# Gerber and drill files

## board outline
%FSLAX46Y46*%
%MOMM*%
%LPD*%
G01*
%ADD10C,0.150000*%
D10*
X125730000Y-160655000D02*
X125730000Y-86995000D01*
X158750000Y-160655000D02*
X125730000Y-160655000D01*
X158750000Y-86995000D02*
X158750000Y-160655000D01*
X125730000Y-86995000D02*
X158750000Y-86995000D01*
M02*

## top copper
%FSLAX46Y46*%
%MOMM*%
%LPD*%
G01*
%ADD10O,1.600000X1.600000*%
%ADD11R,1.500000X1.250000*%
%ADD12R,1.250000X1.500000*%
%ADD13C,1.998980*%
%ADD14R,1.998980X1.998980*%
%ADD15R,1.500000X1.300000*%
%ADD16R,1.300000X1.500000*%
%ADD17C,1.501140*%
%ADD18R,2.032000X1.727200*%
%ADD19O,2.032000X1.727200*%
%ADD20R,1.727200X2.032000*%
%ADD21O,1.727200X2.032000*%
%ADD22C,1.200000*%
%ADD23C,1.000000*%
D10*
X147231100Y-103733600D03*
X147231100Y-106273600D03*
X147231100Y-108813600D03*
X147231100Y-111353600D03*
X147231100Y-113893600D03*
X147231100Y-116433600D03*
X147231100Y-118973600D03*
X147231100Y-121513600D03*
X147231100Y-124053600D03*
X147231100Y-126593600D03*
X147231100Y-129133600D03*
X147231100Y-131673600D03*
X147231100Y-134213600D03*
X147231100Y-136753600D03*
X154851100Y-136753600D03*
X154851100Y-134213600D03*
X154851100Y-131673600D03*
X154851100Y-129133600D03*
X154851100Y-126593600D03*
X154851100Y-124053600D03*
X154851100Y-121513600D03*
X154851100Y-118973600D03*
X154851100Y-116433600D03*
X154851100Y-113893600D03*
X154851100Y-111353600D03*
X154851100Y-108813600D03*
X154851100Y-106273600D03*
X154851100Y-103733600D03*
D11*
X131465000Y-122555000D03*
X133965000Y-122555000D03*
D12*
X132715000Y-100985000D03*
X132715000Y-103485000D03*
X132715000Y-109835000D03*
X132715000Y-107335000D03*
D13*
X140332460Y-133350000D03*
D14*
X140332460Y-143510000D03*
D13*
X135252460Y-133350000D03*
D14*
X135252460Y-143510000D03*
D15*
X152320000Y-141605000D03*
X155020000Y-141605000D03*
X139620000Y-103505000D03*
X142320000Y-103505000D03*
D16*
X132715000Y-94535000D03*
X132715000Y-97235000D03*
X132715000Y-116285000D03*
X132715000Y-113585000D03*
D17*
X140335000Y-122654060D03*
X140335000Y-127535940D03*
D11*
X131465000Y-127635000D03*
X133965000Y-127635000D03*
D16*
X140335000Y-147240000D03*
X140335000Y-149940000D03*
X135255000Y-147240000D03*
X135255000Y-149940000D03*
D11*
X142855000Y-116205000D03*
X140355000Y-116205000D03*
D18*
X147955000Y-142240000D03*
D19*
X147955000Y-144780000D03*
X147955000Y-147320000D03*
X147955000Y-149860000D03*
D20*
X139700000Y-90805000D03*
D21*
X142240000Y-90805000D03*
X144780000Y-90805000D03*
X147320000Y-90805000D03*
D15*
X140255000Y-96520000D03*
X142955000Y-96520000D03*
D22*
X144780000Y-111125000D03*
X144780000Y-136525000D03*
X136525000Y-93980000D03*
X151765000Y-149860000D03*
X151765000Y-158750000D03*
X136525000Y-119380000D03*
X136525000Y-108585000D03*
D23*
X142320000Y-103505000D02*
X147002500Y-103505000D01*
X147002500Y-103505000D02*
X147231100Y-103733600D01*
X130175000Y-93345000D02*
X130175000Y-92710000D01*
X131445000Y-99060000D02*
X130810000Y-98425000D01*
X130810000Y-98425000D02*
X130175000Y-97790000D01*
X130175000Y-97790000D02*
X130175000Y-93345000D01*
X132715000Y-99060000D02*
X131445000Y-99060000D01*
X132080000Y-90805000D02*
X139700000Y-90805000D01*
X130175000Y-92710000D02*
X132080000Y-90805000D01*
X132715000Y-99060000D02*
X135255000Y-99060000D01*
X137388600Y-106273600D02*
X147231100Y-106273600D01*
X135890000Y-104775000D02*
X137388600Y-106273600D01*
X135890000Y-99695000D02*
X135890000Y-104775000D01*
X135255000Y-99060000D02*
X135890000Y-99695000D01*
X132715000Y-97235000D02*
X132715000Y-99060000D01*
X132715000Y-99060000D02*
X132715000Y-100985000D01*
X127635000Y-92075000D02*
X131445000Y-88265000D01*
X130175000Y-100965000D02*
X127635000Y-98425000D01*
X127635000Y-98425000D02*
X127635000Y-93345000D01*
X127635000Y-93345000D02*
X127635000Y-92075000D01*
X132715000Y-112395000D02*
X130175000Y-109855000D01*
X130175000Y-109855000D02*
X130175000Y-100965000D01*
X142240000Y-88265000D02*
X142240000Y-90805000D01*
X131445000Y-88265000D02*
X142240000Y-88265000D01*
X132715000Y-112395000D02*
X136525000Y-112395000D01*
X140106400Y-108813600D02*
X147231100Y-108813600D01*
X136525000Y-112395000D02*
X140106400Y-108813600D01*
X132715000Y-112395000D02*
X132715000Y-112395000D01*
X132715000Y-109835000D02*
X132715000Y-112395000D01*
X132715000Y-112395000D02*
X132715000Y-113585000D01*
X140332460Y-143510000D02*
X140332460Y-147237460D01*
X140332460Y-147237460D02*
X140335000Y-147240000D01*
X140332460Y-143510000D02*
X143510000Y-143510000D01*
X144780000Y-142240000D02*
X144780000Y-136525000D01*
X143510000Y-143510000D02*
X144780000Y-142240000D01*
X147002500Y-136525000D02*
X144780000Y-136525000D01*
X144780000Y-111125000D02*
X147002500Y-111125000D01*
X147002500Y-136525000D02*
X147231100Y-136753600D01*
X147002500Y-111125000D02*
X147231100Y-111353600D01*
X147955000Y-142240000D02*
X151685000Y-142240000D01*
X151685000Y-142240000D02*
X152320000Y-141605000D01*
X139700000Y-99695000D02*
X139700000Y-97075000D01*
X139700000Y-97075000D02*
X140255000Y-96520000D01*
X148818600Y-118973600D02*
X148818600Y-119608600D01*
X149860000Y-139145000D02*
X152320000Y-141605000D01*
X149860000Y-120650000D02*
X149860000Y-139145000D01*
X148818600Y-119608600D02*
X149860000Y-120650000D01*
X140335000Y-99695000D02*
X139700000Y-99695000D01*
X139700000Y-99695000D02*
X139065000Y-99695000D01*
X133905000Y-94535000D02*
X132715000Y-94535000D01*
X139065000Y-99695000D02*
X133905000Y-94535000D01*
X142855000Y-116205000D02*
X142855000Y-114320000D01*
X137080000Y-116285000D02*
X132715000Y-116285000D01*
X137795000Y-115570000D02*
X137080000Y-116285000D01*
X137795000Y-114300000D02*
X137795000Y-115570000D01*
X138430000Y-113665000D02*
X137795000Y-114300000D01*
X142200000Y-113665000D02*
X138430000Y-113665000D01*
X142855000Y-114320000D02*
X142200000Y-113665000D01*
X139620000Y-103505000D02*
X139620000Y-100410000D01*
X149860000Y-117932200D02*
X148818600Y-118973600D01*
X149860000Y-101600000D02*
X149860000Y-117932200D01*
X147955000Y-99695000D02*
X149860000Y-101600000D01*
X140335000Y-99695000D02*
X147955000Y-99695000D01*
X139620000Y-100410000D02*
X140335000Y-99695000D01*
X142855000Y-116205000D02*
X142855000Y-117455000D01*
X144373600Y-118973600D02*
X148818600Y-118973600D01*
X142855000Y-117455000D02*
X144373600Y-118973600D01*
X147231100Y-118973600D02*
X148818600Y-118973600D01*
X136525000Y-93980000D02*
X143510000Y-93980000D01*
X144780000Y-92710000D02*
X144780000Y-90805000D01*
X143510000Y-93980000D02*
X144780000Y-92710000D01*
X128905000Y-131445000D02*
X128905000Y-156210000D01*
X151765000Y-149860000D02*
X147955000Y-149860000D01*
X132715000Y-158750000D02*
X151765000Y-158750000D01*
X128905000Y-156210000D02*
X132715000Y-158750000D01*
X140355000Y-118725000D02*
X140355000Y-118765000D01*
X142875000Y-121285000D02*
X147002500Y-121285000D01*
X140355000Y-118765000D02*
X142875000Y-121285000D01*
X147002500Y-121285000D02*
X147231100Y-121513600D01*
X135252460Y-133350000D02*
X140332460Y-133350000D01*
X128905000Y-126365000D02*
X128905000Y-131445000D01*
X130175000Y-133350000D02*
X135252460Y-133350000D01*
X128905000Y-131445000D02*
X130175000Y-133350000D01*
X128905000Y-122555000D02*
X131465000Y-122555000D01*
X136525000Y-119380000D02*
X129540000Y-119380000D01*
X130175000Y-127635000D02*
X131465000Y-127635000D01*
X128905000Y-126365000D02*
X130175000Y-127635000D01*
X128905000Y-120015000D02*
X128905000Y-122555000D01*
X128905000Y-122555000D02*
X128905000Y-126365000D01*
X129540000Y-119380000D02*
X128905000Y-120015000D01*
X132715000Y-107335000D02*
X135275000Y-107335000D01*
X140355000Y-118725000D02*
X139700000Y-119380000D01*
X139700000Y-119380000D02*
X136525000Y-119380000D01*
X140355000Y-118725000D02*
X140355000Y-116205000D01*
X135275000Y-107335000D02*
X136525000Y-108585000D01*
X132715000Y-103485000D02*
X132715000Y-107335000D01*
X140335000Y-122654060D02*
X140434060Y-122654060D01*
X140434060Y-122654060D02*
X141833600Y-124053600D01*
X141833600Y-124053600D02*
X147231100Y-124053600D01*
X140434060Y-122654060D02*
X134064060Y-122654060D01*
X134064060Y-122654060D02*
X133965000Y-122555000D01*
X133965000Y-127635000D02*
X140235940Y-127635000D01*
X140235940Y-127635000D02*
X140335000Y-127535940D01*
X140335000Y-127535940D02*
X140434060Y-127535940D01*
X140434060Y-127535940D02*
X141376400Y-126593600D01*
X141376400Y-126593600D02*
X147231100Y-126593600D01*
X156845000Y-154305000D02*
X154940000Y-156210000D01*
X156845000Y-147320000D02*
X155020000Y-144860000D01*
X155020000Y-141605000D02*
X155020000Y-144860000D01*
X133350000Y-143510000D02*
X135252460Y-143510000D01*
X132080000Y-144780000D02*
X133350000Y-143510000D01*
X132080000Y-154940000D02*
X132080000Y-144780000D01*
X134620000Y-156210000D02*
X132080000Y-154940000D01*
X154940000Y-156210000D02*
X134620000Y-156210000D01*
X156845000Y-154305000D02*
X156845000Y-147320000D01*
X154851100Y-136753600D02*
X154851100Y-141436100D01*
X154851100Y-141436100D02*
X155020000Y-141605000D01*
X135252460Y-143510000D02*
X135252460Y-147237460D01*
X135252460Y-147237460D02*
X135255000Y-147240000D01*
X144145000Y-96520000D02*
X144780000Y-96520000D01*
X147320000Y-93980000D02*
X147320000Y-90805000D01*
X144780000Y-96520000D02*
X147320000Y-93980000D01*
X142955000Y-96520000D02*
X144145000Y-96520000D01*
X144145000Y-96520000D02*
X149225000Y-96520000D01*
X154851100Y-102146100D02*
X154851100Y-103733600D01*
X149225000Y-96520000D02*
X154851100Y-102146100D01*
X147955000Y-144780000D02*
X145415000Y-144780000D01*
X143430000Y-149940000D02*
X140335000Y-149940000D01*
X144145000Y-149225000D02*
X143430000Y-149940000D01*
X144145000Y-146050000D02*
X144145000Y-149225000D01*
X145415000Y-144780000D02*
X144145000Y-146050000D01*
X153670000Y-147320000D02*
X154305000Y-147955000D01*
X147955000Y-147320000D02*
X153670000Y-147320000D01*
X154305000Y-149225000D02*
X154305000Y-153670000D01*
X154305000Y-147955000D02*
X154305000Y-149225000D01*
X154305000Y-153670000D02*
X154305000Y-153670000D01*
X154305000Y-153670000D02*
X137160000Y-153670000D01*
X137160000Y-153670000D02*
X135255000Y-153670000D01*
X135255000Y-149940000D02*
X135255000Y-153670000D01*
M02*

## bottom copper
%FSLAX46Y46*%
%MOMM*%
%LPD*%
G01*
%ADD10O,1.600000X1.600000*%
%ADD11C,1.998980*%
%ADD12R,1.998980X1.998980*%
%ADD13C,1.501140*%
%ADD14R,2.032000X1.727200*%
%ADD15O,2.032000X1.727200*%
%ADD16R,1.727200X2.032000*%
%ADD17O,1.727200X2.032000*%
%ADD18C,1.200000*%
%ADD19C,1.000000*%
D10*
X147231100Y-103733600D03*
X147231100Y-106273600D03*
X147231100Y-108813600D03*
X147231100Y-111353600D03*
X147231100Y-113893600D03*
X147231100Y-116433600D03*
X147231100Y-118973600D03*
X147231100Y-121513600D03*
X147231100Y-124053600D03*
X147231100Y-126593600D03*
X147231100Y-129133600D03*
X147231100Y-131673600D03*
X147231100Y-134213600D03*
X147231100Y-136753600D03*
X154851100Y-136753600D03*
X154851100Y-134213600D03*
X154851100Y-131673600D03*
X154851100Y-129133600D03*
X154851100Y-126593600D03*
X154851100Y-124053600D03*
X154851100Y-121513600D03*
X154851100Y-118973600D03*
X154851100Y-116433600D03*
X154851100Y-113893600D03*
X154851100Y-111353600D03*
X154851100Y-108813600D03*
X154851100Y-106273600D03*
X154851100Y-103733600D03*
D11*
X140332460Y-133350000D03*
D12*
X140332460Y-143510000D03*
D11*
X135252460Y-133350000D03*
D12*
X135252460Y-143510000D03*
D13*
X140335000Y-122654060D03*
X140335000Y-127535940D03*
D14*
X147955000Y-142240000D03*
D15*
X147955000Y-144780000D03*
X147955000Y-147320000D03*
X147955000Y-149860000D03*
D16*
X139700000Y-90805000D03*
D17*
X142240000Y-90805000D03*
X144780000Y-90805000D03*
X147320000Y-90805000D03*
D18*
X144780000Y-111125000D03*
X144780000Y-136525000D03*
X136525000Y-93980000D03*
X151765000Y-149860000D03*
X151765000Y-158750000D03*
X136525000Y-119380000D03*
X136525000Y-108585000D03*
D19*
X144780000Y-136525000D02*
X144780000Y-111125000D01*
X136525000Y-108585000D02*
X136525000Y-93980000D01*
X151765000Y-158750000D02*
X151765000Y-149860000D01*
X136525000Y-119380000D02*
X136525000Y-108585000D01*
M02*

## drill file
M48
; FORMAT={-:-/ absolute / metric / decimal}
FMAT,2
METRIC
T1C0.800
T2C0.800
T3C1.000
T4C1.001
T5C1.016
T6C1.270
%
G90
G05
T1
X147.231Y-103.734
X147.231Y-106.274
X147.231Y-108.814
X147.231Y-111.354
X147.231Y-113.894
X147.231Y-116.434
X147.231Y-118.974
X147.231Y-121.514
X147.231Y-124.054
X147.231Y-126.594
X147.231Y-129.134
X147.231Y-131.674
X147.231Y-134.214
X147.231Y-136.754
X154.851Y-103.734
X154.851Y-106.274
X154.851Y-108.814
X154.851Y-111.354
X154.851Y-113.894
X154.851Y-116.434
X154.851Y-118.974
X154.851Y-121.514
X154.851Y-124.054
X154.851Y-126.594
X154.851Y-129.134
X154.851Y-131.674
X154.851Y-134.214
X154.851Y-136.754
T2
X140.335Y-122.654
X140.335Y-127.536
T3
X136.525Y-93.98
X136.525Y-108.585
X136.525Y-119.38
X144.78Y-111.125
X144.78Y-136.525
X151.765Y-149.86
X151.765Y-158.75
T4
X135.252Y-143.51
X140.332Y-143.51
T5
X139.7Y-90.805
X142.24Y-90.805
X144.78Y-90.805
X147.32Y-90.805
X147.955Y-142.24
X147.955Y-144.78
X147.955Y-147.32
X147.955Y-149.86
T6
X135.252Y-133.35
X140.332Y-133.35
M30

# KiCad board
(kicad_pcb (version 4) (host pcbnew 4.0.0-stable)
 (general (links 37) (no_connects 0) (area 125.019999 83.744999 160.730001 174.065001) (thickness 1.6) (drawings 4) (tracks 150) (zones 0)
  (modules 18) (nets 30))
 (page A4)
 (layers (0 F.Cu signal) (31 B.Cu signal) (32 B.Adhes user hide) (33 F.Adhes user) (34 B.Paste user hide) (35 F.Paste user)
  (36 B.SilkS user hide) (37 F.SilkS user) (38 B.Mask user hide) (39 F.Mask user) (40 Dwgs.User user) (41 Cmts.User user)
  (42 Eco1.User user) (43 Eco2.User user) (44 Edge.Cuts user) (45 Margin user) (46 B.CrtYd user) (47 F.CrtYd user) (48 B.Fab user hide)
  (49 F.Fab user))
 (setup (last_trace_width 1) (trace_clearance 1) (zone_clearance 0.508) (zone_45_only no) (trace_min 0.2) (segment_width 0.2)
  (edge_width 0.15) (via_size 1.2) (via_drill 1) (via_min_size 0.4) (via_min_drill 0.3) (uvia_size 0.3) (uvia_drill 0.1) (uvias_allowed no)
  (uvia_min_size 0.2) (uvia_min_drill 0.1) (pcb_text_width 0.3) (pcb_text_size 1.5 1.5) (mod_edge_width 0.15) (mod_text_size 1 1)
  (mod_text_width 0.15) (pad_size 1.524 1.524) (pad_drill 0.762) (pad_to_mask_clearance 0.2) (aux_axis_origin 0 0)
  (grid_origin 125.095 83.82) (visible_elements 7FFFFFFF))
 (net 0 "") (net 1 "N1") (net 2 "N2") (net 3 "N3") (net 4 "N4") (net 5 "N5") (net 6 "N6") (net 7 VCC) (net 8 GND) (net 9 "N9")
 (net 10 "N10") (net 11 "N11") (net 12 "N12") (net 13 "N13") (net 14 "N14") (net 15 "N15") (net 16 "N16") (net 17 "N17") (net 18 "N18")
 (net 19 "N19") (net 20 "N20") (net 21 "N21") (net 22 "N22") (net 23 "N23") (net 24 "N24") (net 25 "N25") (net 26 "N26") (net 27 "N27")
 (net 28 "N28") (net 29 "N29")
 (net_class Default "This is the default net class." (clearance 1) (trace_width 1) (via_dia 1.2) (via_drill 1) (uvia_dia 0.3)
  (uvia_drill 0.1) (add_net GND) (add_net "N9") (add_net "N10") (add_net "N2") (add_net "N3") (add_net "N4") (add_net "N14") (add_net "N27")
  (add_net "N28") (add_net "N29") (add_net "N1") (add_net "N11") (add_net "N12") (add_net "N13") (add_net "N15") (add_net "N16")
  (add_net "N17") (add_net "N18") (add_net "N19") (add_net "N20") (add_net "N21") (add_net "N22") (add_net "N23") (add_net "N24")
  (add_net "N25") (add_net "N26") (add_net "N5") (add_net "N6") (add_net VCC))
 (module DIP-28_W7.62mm (layer F.Cu) (at 147.2311 103.7336)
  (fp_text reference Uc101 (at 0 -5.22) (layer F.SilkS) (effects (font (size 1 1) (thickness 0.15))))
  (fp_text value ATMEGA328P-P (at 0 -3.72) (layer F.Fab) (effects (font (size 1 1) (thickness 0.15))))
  (pad 1 thru_hole oval (at 0 0) (size 1.6 1.6) (drill 0.8) (layers *.Cu *.Mask F.SilkS) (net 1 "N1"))
  (pad 2 thru_hole oval (at 0 2.54) (size 1.6 1.6) (drill 0.8) (layers *.Cu *.Mask F.SilkS) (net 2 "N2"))
  (pad 3 thru_hole oval (at 0 5.08) (size 1.6 1.6) (drill 0.8) (layers *.Cu *.Mask F.SilkS) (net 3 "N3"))
  (pad 4 thru_hole oval (at 0 7.62) (size 1.6 1.6) (drill 0.8) (layers *.Cu *.Mask F.SilkS) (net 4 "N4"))
  (pad 5 thru_hole oval (at 0 10.16) (size 1.6 1.6) (drill 0.8) (layers *.Cu *.Mask F.SilkS) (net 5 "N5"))
  (pad 6 thru_hole oval (at 0 12.7) (size 1.6 1.6) (drill 0.8) (layers *.Cu *.Mask F.SilkS) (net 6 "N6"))
  (pad 7 thru_hole oval (at 0 15.24) (size 1.6 1.6) (drill 0.8) (layers *.Cu *.Mask F.SilkS) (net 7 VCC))
  (pad 8 thru_hole oval (at 0 17.78) (size 1.6 1.6) (drill 0.8) (layers *.Cu *.Mask F.SilkS) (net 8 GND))
  (pad 9 thru_hole oval (at 0 20.32) (size 1.6 1.6) (drill 0.8) (layers *.Cu *.Mask F.SilkS) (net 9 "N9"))
  (pad 10 thru_hole oval (at 0 22.86) (size 1.6 1.6) (drill 0.8) (layers *.Cu *.Mask F.SilkS) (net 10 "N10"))
  (pad 11 thru_hole oval (at 0 25.4) (size 1.6 1.6) (drill 0.8) (layers *.Cu *.Mask F.SilkS) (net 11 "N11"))
  (pad 12 thru_hole oval (at 0 27.94) (size 1.6 1.6) (drill 0.8) (layers *.Cu *.Mask F.SilkS) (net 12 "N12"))
  (pad 13 thru_hole oval (at 0 30.48) (size 1.6 1.6) (drill 0.8) (layers *.Cu *.Mask F.SilkS) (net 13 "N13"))
  (pad 14 thru_hole oval (at 0 33.02) (size 1.6 1.6) (drill 0.8) (layers *.Cu *.Mask F.SilkS) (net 4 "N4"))
  (pad 15 thru_hole oval (at 7.62 33.02) (size 1.6 1.6) (drill 0.8) (layers *.Cu *.Mask F.SilkS) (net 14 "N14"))
  (pad 16 thru_hole oval (at 7.62 30.48) (size 1.6 1.6) (drill 0.8) (layers *.Cu *.Mask F.SilkS) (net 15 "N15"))
  (pad 17 thru_hole oval (at 7.62 27.94) (size 1.6 1.6) (drill 0.8) (layers *.Cu *.Mask F.SilkS) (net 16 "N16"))
  (pad 18 thru_hole oval (at 7.62 25.4) (size 1.6 1.6) (drill 0.8) (layers *.Cu *.Mask F.SilkS) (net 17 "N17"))
  (pad 19 thru_hole oval (at 7.62 22.86) (size 1.6 1.6) (drill 0.8) (layers *.Cu *.Mask F.SilkS) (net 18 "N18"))
  (pad 20 thru_hole oval (at 7.62 20.32) (size 1.6 1.6) (drill 0.8) (layers *.Cu *.Mask F.SilkS) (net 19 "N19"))
  (pad 21 thru_hole oval (at 7.62 17.78) (size 1.6 1.6) (drill 0.8) (layers *.Cu *.Mask F.SilkS) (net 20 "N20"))
  (pad 22 thru_hole oval (at 7.62 15.24) (size 1.6 1.6) (drill 0.8) (layers *.Cu *.Mask F.SilkS) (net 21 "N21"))
  (pad 23 thru_hole oval (at 7.62 12.7) (size 1.6 1.6) (drill 0.8) (layers *.Cu *.Mask F.SilkS) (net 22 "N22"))
  (pad 24 thru_hole oval (at 7.62 10.16) (size 1.6 1.6) (drill 0.8) (layers *.Cu *.Mask F.SilkS) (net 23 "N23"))
  (pad 25 thru_hole oval (at 7.62 7.62) (size 1.6 1.6) (drill 0.8) (layers *.Cu *.Mask F.SilkS) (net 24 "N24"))
  (pad 26 thru_hole oval (at 7.62 5.08) (size 1.6 1.6) (drill 0.8) (layers *.Cu *.Mask F.SilkS) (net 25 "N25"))
  (pad 27 thru_hole oval (at 7.62 2.54) (size 1.6 1.6) (drill 0.8) (layers *.Cu *.Mask F.SilkS) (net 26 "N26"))
  (pad 28 thru_hole oval (at 7.62 0) (size 1.6 1.6) (drill 0.8) (layers *.Cu *.Mask F.SilkS) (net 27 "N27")))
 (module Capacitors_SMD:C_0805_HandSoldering (layer F.Cu) (at 132.715 122.555)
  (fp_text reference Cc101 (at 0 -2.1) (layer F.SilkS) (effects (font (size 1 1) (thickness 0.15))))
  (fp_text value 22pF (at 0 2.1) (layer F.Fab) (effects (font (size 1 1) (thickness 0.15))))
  (pad 1 smd rect (at -1.25 0) (size 1.5 1.25) (layers F.Cu F.Paste F.Mask) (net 8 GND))
  (pad 2 smd rect (at 1.25 0) (size 1.5 1.25) (layers F.Cu F.Paste F.Mask) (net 9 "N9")))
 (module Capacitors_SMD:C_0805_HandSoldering (layer F.Cu) (at 132.715 102.235 270)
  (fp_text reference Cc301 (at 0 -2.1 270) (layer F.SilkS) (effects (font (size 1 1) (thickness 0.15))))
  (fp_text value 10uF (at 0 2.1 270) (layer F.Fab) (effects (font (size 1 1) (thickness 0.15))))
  (pad 1 smd rect (at -1.25 0 270) (size 1.5 1.25) (layers F.Cu F.Paste F.Mask) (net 2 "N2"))
  (pad 2 smd rect (at 1.25 0 270) (size 1.5 1.25) (layers F.Cu F.Paste F.Mask) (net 8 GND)))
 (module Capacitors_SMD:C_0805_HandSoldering (layer F.Cu) (at 132.715 108.585 90)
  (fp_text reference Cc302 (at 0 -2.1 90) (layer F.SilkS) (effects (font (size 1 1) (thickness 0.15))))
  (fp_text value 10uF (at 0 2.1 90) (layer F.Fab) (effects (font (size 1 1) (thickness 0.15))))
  (pad 1 smd rect (at -1.25 0 90) (size 1.5 1.25) (layers F.Cu F.Paste F.Mask) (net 3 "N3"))
  (pad 2 smd rect (at 1.25 0 90) (size 1.5 1.25) (layers F.Cu F.Paste F.Mask) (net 8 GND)))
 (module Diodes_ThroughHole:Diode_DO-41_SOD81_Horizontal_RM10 (layer F.Cu) (at 140.335 143.51 90)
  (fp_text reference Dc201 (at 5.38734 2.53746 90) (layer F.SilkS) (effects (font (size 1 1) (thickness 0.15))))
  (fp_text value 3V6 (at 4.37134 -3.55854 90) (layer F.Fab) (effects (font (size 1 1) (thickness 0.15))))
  (pad 2 thru_hole circle (at 10.16 -0.00254 270) (size 1.99898 1.99898) (drill 1.27) (layers *.Cu *.Mask F.SilkS) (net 8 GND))
  (pad 1 thru_hole rect (at 0 -0.00254 270) (size 1.99898 1.99898) (drill 1.00076) (layers *.Cu *.Mask F.SilkS) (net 4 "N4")))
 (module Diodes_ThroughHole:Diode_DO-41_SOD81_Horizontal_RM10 (layer F.Cu) (at 135.255 143.51 90)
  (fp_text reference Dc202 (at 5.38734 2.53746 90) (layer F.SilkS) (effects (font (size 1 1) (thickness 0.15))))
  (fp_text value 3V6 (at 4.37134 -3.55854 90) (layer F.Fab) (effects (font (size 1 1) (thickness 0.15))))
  (pad 2 thru_hole circle (at 10.16 -0.00254 270) (size 1.99898 1.99898) (drill 1.27) (layers *.Cu *.Mask F.SilkS) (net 8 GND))
  (pad 1 thru_hole rect (at 0 -0.00254 270) (size 1.99898 1.99898) (drill 1.00076) (layers *.Cu *.Mask F.SilkS) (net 14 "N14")))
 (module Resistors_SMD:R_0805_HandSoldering (layer F.Cu) (at 153.67 141.605)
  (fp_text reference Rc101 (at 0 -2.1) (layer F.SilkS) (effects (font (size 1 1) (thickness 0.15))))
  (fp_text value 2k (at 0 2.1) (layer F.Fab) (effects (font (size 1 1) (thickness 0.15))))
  (pad 1 smd rect (at -1.35 0) (size 1.5 1.3) (layers F.Cu F.Paste F.Mask) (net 7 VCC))
  (pad 2 smd rect (at 1.35 0) (size 1.5 1.3) (layers F.Cu F.Paste F.Mask) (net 14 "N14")))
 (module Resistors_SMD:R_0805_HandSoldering (layer F.Cu) (at 140.97 103.505)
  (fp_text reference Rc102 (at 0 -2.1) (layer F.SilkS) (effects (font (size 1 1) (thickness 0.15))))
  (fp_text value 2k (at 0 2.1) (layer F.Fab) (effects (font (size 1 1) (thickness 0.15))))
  (pad 1 smd rect (at -1.35 0) (size 1.5 1.3) (layers F.Cu F.Paste F.Mask) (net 7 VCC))
  (pad 2 smd rect (at 1.35 0) (size 1.5 1.3) (layers F.Cu F.Paste F.Mask) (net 1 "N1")))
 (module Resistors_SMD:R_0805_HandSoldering (layer F.Cu) (at 132.715 95.885 270)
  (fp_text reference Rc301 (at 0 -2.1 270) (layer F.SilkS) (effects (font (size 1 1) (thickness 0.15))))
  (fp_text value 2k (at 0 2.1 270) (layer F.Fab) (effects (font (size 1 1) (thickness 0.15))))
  (pad 1 smd rect (at -1.35 0 270) (size 1.5 1.3) (layers F.Cu F.Paste F.Mask) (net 7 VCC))
  (pad 2 smd rect (at 1.35 0 270) (size 1.5 1.3) (layers F.Cu F.Paste F.Mask) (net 2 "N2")))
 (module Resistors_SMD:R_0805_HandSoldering (layer F.Cu) (at 132.715 114.935 90)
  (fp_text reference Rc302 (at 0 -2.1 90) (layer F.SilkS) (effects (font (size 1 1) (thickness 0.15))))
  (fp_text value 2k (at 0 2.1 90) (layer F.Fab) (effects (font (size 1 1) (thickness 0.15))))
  (pad 1 smd rect (at -1.35 0 90) (size 1.5 1.3) (layers F.Cu F.Paste F.Mask) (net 7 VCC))
  (pad 2 smd rect (at 1.35 0 90) (size 1.5 1.3) (layers F.Cu F.Paste F.Mask) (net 3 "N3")))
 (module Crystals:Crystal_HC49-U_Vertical (layer F.Cu) (at 140.335 125.095 270)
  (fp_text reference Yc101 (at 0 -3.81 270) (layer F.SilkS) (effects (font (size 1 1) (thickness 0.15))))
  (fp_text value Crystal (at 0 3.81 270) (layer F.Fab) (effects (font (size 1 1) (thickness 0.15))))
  (pad 1 thru_hole circle (at -2.44094 0 270) (size 1.50114 1.50114) (drill 0.8001) (layers *.Cu *.Mask F.SilkS) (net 9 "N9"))
  (pad 2 thru_hole circle (at 2.44094 0 270) (size 1.50114 1.50114) (drill 0.8001) (layers *.Cu *.Mask F.SilkS) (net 10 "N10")))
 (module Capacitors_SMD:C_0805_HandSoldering (layer F.Cu) (at 132.715 127.635)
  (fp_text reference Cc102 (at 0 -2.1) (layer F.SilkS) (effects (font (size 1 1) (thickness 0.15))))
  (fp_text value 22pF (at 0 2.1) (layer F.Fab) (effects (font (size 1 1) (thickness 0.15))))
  (pad 1 smd rect (at -1.25 0) (size 1.5 1.25) (layers F.Cu F.Paste F.Mask) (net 8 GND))
  (pad 2 smd rect (at 1.25 0) (size 1.5 1.25) (layers F.Cu F.Paste F.Mask) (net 10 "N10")))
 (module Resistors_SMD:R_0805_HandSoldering (layer F.Cu) (at 140.335 148.59 270)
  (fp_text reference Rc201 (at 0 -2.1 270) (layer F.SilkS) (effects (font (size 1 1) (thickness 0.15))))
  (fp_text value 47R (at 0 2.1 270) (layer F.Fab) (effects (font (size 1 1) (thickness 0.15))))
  (pad 1 smd rect (at -1.35 0 270) (size 1.5 1.3) (layers F.Cu F.Paste F.Mask) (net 4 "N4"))
  (pad 2 smd rect (at 1.35 0 270) (size 1.5 1.3) (layers F.Cu F.Paste F.Mask) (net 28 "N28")))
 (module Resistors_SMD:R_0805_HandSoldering (layer F.Cu) (at 135.255 148.59 270)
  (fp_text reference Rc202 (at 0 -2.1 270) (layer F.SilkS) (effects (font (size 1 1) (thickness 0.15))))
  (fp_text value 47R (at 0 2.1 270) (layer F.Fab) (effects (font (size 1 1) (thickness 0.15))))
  (pad 1 smd rect (at -1.35 0 270) (size 1.5 1.3) (layers F.Cu F.Paste F.Mask) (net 14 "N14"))
  (pad 2 smd rect (at 1.35 0 270) (size 1.5 1.3) (layers F.Cu F.Paste F.Mask) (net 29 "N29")))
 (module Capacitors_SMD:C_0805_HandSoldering (layer F.Cu) (at 141.605 116.205 180)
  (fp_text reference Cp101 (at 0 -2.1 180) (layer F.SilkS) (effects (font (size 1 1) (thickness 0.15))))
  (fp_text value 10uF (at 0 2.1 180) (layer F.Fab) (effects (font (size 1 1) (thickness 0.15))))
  (pad 1 smd rect (at -1.25 0 180) (size 1.5 1.25) (layers F.Cu F.Paste F.Mask) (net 7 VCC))
  (pad 2 smd rect (at 1.25 0 180) (size 1.5 1.25) (layers F.Cu F.Paste F.Mask) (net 8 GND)))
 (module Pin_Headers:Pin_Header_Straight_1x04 (layer F.Cu) (at 147.955 142.24)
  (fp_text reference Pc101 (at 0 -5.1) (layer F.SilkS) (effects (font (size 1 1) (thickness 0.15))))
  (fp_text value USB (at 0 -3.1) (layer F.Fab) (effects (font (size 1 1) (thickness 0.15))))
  (pad 1 thru_hole rect (at 0 0) (size 2.032 1.7272) (drill 1.016) (layers *.Cu *.Mask F.SilkS) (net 7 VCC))
  (pad 2 thru_hole oval (at 0 2.54) (size 2.032 1.7272) (drill 1.016) (layers *.Cu *.Mask F.SilkS) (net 28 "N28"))
  (pad 3 thru_hole oval (at 0 5.08) (size 2.032 1.7272) (drill 1.016) (layers *.Cu *.Mask F.SilkS) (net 29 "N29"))
  (pad 4 thru_hole oval (at 0 7.62) (size 2.032 1.7272) (drill 1.016) (layers *.Cu *.Mask F.SilkS) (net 8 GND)))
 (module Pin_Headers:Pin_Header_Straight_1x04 (layer F.Cu) (at 139.7 90.805 90)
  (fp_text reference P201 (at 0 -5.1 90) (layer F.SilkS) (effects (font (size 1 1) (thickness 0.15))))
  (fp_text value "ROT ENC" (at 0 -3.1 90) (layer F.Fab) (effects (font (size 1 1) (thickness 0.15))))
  (pad 1 thru_hole rect (at 0 0 90) (size 2.032 1.7272) (drill 1.016) (layers *.Cu *.Mask F.SilkS) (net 2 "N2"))
  (pad 2 thru_hole oval (at 0 2.54 90) (size 2.032 1.7272) (drill 1.016) (layers *.Cu *.Mask F.SilkS) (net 3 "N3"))
  (pad 3 thru_hole oval (at 0 5.08 90) (size 2.032 1.7272) (drill 1.016) (layers *.Cu *.Mask F.SilkS) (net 8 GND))
  (pad 4 thru_hole oval (at 0 7.62 90) (size 2.032 1.7272) (drill 1.016) (layers *.Cu *.Mask F.SilkS) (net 27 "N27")))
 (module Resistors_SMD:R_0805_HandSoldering (layer F.Cu) (at 141.605 96.52)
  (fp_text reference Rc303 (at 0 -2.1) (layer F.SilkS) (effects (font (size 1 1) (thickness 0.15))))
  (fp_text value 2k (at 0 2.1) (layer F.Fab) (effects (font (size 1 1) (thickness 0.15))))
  (pad 1 smd rect (at -1.35 0) (size 1.5 1.3) (layers F.Cu F.Paste F.Mask) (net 7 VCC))
  (pad 2 smd rect (at 1.35 0) (size 1.5 1.3) (layers F.Cu F.Paste F.Mask) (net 27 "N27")))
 (gr_line (start 125.73 160.655) (end 125.73 86.995) (angle 90) (layer Edge.Cuts) (width 0.15))
 (gr_line (start 158.75 160.655) (end 125.73 160.655) (angle 90) (layer Edge.Cuts) (width 0.15))
 (gr_line (start 158.75 86.995) (end 158.75 160.655) (angle 90) (layer Edge.Cuts) (width 0.15))
 (gr_line (start 125.73 86.995) (end 158.75 86.995) (angle 90) (layer Edge.Cuts) (width 0.15))
 (segment (start 142.32 103.505) (end 147.0025 103.505) (width 1) (layer F.Cu) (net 1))
 (segment (start 147.0025 103.505) (end 147.2311 103.7336) (width 1) (layer F.Cu) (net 1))
 (segment (start 130.175 93.345) (end 130.175 92.71) (width 1) (layer F.Cu) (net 2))
 (segment (start 131.445 99.06) (end 130.81 98.425) (width 1) (layer F.Cu) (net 2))
 (segment (start 130.81 98.425) (end 130.175 97.79) (width 1) (layer F.Cu) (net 2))
 (segment (start 130.175 97.79) (end 130.175 93.345) (width 1) (layer F.Cu) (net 2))
 (segment (start 132.715 99.06) (end 131.445 99.06) (width 1) (layer F.Cu) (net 2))
 (segment (start 132.08 90.805) (end 139.7 90.805) (width 1) (layer F.Cu) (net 2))
 (segment (start 130.175 92.71) (end 132.08 90.805) (width 1) (layer F.Cu) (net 2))
 (segment (start 132.715 99.06) (end 135.255 99.06) (width 1) (layer F.Cu) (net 2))
 (segment (start 137.3886 106.2736) (end 147.2311 106.2736) (width 1) (layer F.Cu) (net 2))
 (segment (start 135.89 104.775) (end 137.3886 106.2736) (width 1) (layer F.Cu) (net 2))
 (segment (start 135.89 99.695) (end 135.89 104.775) (width 1) (layer F.Cu) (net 2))
 (segment (start 135.255 99.06) (end 135.89 99.695) (width 1) (layer F.Cu) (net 2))
 (segment (start 132.715 97.235) (end 132.715 99.06) (width 1) (layer F.Cu) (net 2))
 (segment (start 132.715 99.06) (end 132.715 100.985) (width 1) (layer F.Cu) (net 2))
 (segment (start 127.635 92.075) (end 131.445 88.265) (width 1) (layer F.Cu) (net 3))
 (segment (start 130.175 100.965) (end 127.635 98.425) (width 1) (layer F.Cu) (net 3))
 (segment (start 127.635 98.425) (end 127.635 93.345) (width 1) (layer F.Cu) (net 3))
 (segment (start 127.635 93.345) (end 127.635 92.075) (width 1) (layer F.Cu) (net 3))
 (segment (start 132.715 112.395) (end 130.175 109.855) (width 1) (layer F.Cu) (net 3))
 (segment (start 130.175 109.855) (end 130.175 100.965) (width 1) (layer F.Cu) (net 3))
 (segment (start 142.24 88.265) (end 142.24 90.805) (width 1) (layer F.Cu) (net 3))
 (segment (start 131.445 88.265) (end 142.24 88.265) (width 1) (layer F.Cu) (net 3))
 (segment (start 132.715 112.395) (end 136.525 112.395) (width 1) (layer F.Cu) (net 3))
 (segment (start 140.1064 108.8136) (end 147.2311 108.8136) (width 1) (layer F.Cu) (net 3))
 (segment (start 136.525 112.395) (end 140.1064 108.8136) (width 1) (layer F.Cu) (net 3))
 (segment (start 132.715 112.395) (end 132.715 112.395) (width 1) (layer F.Cu) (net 3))
 (segment (start 132.715 109.835) (end 132.715 112.395) (width 1) (layer F.Cu) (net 3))
 (segment (start 132.715 112.395) (end 132.715 113.585) (width 1) (layer F.Cu) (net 3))
 (segment (start 140.33246 143.51) (end 140.33246 147.23746) (width 1) (layer F.Cu) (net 4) (status 20))
 (segment (start 140.33246 147.23746) (end 140.335 147.24) (width 1) (layer F.Cu) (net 4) (status 30))
 (segment (start 140.33246 143.51) (end 143.51 143.51) (width 1) (layer F.Cu) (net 4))
 (segment (start 144.78 142.24) (end 144.78 136.525) (width 1) (layer F.Cu) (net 4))
 (segment (start 143.51 143.51) (end 144.78 142.24) (width 1) (layer F.Cu) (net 4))
 (segment (start 147.0025 136.525) (end 144.78 136.525) (width 1) (layer F.Cu) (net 4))
 (via (at 144.78 111.125) (size 1.2) (drill 1) (layers F.Cu B.Cu) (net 4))
 (segment (start 144.78 136.525) (end 144.78 111.125) (width 1) (layer B.Cu) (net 4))
 (via (at 144.78 136.525) (size 1.2) (drill 1) (layers F.Cu B.Cu) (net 4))
 (segment (start 144.78 111.125) (end 147.0025 111.125) (width 1) (layer F.Cu) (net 4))
 (segment (start 147.0025 136.525) (end 147.2311 136.7536) (width 1) (layer F.Cu) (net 4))
 (segment (start 147.0025 111.125) (end 147.2311 111.3536) (width 1) (layer F.Cu) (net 4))
 (segment (start 147.955 142.24) (end 151.685 142.24) (width 1) (layer F.Cu) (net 7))
 (segment (start 151.685 142.24) (end 152.32 141.605) (width 1) (layer F.Cu) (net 7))
 (segment (start 139.7 99.695) (end 139.7 97.075) (width 1) (layer F.Cu) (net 7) (status 20))
 (segment (start 139.7 97.075) (end 140.255 96.52) (width 1) (layer F.Cu) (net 7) (status 30))
 (segment (start 148.8186 118.9736) (end 148.8186 119.6086) (width 1) (layer F.Cu) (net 7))
 (segment (start 149.86 139.145) (end 152.32 141.605) (width 1) (layer F.Cu) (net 7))
 (segment (start 149.86 120.65) (end 149.86 139.145) (width 1) (layer F.Cu) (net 7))
 (segment (start 148.8186 119.6086) (end 149.86 120.65) (width 1) (layer F.Cu) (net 7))
 (segment (start 140.335 99.695) (end 139.7 99.695) (width 1) (layer F.Cu) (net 7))
 (segment (start 139.7 99.695) (end 139.065 99.695) (width 1) (layer F.Cu) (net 7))
 (segment (start 133.905 94.535) (end 132.715 94.535) (width 1) (layer F.Cu) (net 7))
 (segment (start 139.065 99.695) (end 133.905 94.535) (width 1) (layer F.Cu) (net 7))
 (segment (start 142.855 116.205) (end 142.855 114.32) (width 1) (layer F.Cu) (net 7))
 (segment (start 137.08 116.285) (end 132.715 116.285) (width 1) (layer F.Cu) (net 7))
 (segment (start 137.795 115.57) (end 137.08 116.285) (width 1) (layer F.Cu) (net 7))
 (segment (start 137.795 114.3) (end 137.795 115.57) (width 1) (layer F.Cu) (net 7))
 (segment (start 138.43 113.665) (end 137.795 114.3) (width 1) (layer F.Cu) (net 7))
 (segment (start 142.2 113.665) (end 138.43 113.665) (width 1) (layer F.Cu) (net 7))
 (segment (start 142.855 114.32) (end 142.2 113.665) (width 1) (layer F.Cu) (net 7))
 (segment (start 139.62 103.505) (end 139.62 100.41) (width 1) (layer F.Cu) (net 7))
 (segment (start 149.86 117.9322) (end 148.8186 118.9736) (width 1) (layer F.Cu) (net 7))
 (segment (start 149.86 101.6) (end 149.86 117.9322) (width 1) (layer F.Cu) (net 7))
 (segment (start 147.955 99.695) (end 149.86 101.6) (width 1) (layer F.Cu) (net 7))
 (segment (start 140.335 99.695) (end 147.955 99.695) (width 1) (layer F.Cu) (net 7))
 (segment (start 139.62 100.41) (end 140.335 99.695) (width 1) (layer F.Cu) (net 7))
 (segment (start 142.855 116.205) (end 142.855 117.455) (width 1) (layer F.Cu) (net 7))
 (segment (start 144.3736 118.9736) (end 148.8186 118.9736) (width 1) (layer F.Cu) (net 7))
 (segment (start 142.855 117.455) (end 144.3736 118.9736) (width 1) (layer F.Cu) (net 7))
 (segment (start 147.2311 118.9736) (end 148.8186 118.9736) (width 1) (layer F.Cu) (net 7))
 (segment (start 136.525 93.98) (end 143.51 93.98) (width 1) (layer F.Cu) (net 8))
 (via (at 136.525 93.98) (size 1.2) (drill 1) (layers F.Cu B.Cu) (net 8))
 (segment (start 136.525 108.585) (end 136.525 93.98) (width 1) (layer B.Cu) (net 8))
 (segment (start 144.78 92.71) (end 144.78 90.805) (width 1) (layer F.Cu) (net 8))
 (segment (start 143.51 93.98) (end 144.78 92.71) (width 1) (layer F.Cu) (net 8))
 (segment (start 128.905 131.445) (end 128.905 156.21) (width 1) (layer F.Cu) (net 8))
 (segment (start 151.765 149.86) (end 147.955 149.86) (width 1) (layer F.Cu) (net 8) (status 800020))
 (via (at 151.765 149.86) (size 1.2) (drill 1) (layers F.Cu B.Cu) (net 8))
 (segment (start 151.765 158.75) (end 151.765 149.86) (width 1) (layer B.Cu) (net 8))
 (via (at 151.765 158.75) (size 1.2) (drill 1) (layers F.Cu B.Cu) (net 8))
 (segment (start 132.715 158.75) (end 151.765 158.75) (width 1) (layer F.Cu) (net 8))
 (segment (start 128.905 156.21) (end 132.715 158.75) (width 1) (layer F.Cu) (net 8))
 (segment (start 140.355 118.725) (end 140.355 118.765) (width 1) (layer F.Cu) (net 8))
 (segment (start 142.875 121.285) (end 147.0025 121.285) (width 1) (layer F.Cu) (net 8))
 (segment (start 140.355 118.765) (end 142.875 121.285) (width 1) (layer F.Cu) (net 8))
 (segment (start 147.0025 121.285) (end 147.2311 121.5136) (width 1) (layer F.Cu) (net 8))
 (segment (start 135.25246 133.35) (end 140.33246 133.35) (width 1) (layer F.Cu) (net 8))
 (segment (start 128.905 126.365) (end 128.905 131.445) (width 1) (layer F.Cu) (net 8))
 (segment (start 130.175 133.35) (end 135.25246 133.35) (width 1) (layer F.Cu) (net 8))
 (segment (start 128.905 131.445) (end 130.175 133.35) (width 1) (layer F.Cu) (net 8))
 (segment (start 128.905 122.555) (end 131.465 122.555) (width 1) (layer F.Cu) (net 8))
 (segment (start 136.525 119.38) (end 129.54 119.38) (width 1) (layer F.Cu) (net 8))
 (segment (start 130.175 127.635) (end 131.465 127.635) (width 1) (layer F.Cu) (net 8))
 (segment (start 128.905 126.365) (end 130.175 127.635) (width 1) (layer F.Cu) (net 8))
 (segment (start 128.905 120.015) (end 128.905 122.555) (width 1) (layer F.Cu) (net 8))
 (segment (start 128.905 122.555) (end 128.905 126.365) (width 1) (layer F.Cu) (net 8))
 (segment (start 129.54 119.38) (end 128.905 120.015) (width 1) (layer F.Cu) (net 8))
 (segment (start 132.715 107.335) (end 135.275 107.335) (width 1) (layer F.Cu) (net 8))
 (segment (start 140.355 118.725) (end 139.7 119.38) (width 1) (layer F.Cu) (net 8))
 (segment (start 139.7 119.38) (end 136.525 119.38) (width 1) (layer F.Cu) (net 8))
 (via (at 136.525 119.38) (size 1.2) (drill 1) (layers F.Cu B.Cu) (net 8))
 (segment (start 136.525 119.38) (end 136.525 108.585) (width 1) (layer B.Cu) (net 8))
 (via (at 136.525 108.585) (size 1.2) (drill 1) (layers F.Cu B.Cu) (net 8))
 (segment (start 140.355 118.725) (end 140.355 116.205) (width 1) (layer F.Cu) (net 8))
 (segment (start 135.275 107.335) (end 136.525 108.585) (width 1) (layer F.Cu) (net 8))
 (segment (start 132.715 103.485) (end 132.715 107.335) (width 1) (layer F.Cu) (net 8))
 (segment (start 140.335 122.65406) (end 140.43406 122.65406) (width 1) (layer F.Cu) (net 9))
 (segment (start 140.43406 122.65406) (end 141.8336 124.0536) (width 1) (layer F.Cu) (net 9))
 (segment (start 141.8336 124.0536) (end 147.2311 124.0536) (width 1) (layer F.Cu) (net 9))
 (segment (start 140.43406 122.65406) (end 134.06406 122.65406) (width 1) (layer F.Cu) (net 9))
 (segment (start 134.06406 122.65406) (end 133.965 122.555) (width 1) (layer F.Cu) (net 9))
 (segment (start 133.965 127.635) (end 140.23594 127.635) (width 1) (layer F.Cu) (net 10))
 (segment (start 140.23594 127.635) (end 140.335 127.53594) (width 1) (layer F.Cu) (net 10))
 (segment (start 140.335 127.53594) (end 140.43406 127.53594) (width 1) (layer F.Cu) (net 10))
 (segment (start 140.43406 127.53594) (end 141.3764 126.5936) (width 1) (layer F.Cu) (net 10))
 (segment (start 141.3764 126.5936) (end 147.2311 126.5936) (width 1) (layer F.Cu) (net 10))
 (segment (start 156.845 154.305) (end 154.94 156.21) (width 1) (layer F.Cu) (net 14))
 (segment (start 156.845 147.32) (end 155.02 144.86) (width 1) (layer F.Cu) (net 14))
 (segment (start 155.02 141.605) (end 155.02 144.86) (width 1) (layer F.Cu) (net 14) (status 400000))
 (segment (start 133.35 143.51) (end 135.25246 143.51) (width 1) (layer F.Cu) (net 14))
 (segment (start 132.08 144.78) (end 133.35 143.51) (width 1) (layer F.Cu) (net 14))
 (segment (start 132.08 154.94) (end 132.08 144.78) (width 1) (layer F.Cu) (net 14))
 (segment (start 134.62 156.21) (end 132.08 154.94) (width 1) (layer F.Cu) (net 14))
 (segment (start 154.94 156.21) (end 134.62 156.21) (width 1) (layer F.Cu) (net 14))
 (segment (start 156.845 154.305) (end 156.845 147.32) (width 1) (layer F.Cu) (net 14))
 (segment (start 154.8511 136.7536) (end 154.8511 141.4361) (width 1) (layer F.Cu) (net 14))
 (segment (start 154.8511 141.4361) (end 155.02 141.605) (width 1) (layer F.Cu) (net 14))
 (segment (start 135.25246 143.51) (end 135.25246 147.23746) (width 1) (layer F.Cu) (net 14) (status 20))
 (segment (start 135.25246 147.23746) (end 135.255 147.24) (width 1) (layer F.Cu) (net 14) (status 30))
 (segment (start 144.145 96.52) (end 144.78 96.52) (width 1) (layer F.Cu) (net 27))
 (segment (start 147.32 93.98) (end 147.32 90.805) (width 1) (layer F.Cu) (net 27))
 (segment (start 144.78 96.52) (end 147.32 93.98) (width 1) (layer F.Cu) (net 27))
 (segment (start 142.955 96.52) (end 144.145 96.52) (width 1) (layer F.Cu) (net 27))
 (segment (start 144.145 96.52) (end 149.225 96.52) (width 1) (layer F.Cu) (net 27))
 (segment (start 154.8511 102.1461) (end 154.8511 103.7336) (width 1) (layer F.Cu) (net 27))
 (segment (start 149.225 96.52) (end 154.8511 102.1461) (width 1) (layer F.Cu) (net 27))
 (segment (start 147.955 144.78) (end 145.415 144.78) (width 1) (layer F.Cu) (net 28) (status 400000))
 (segment (start 143.43 149.94) (end 140.335 149.94) (width 1) (layer F.Cu) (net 28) (status 800000))
 (segment (start 144.145 149.225) (end 143.43 149.94) (width 1) (layer F.Cu) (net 28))
 (segment (start 144.145 146.05) (end 144.145 149.225) (width 1) (layer F.Cu) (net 28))
 (segment (start 145.415 144.78) (end 144.145 146.05) (width 1) (layer F.Cu) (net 28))
 (segment (start 153.67 147.32) (end 154.305 147.955) (width 1) (layer F.Cu) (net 29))
 (segment (start 147.955 147.32) (end 153.67 147.32) (width 1) (layer F.Cu) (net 29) (status 400000))
 (segment (start 154.305 149.225) (end 154.305 153.67) (width 1) (layer F.Cu) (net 29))
 (segment (start 154.305 147.955) (end 154.305 149.225) (width 1) (layer F.Cu) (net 29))
 (segment (start 154.305 153.67) (end 154.305 153.67) (width 1) (layer F.Cu) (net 29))
 (segment (start 154.305 153.67) (end 137.16 153.67) (width 1) (layer F.Cu) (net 29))
 (segment (start 137.16 153.67) (end 135.255 153.67) (width 1) (layer F.Cu) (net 29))
 (segment (start 135.255 149.94) (end 135.255 153.67) (width 1) (layer F.Cu) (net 29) (status 20)))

